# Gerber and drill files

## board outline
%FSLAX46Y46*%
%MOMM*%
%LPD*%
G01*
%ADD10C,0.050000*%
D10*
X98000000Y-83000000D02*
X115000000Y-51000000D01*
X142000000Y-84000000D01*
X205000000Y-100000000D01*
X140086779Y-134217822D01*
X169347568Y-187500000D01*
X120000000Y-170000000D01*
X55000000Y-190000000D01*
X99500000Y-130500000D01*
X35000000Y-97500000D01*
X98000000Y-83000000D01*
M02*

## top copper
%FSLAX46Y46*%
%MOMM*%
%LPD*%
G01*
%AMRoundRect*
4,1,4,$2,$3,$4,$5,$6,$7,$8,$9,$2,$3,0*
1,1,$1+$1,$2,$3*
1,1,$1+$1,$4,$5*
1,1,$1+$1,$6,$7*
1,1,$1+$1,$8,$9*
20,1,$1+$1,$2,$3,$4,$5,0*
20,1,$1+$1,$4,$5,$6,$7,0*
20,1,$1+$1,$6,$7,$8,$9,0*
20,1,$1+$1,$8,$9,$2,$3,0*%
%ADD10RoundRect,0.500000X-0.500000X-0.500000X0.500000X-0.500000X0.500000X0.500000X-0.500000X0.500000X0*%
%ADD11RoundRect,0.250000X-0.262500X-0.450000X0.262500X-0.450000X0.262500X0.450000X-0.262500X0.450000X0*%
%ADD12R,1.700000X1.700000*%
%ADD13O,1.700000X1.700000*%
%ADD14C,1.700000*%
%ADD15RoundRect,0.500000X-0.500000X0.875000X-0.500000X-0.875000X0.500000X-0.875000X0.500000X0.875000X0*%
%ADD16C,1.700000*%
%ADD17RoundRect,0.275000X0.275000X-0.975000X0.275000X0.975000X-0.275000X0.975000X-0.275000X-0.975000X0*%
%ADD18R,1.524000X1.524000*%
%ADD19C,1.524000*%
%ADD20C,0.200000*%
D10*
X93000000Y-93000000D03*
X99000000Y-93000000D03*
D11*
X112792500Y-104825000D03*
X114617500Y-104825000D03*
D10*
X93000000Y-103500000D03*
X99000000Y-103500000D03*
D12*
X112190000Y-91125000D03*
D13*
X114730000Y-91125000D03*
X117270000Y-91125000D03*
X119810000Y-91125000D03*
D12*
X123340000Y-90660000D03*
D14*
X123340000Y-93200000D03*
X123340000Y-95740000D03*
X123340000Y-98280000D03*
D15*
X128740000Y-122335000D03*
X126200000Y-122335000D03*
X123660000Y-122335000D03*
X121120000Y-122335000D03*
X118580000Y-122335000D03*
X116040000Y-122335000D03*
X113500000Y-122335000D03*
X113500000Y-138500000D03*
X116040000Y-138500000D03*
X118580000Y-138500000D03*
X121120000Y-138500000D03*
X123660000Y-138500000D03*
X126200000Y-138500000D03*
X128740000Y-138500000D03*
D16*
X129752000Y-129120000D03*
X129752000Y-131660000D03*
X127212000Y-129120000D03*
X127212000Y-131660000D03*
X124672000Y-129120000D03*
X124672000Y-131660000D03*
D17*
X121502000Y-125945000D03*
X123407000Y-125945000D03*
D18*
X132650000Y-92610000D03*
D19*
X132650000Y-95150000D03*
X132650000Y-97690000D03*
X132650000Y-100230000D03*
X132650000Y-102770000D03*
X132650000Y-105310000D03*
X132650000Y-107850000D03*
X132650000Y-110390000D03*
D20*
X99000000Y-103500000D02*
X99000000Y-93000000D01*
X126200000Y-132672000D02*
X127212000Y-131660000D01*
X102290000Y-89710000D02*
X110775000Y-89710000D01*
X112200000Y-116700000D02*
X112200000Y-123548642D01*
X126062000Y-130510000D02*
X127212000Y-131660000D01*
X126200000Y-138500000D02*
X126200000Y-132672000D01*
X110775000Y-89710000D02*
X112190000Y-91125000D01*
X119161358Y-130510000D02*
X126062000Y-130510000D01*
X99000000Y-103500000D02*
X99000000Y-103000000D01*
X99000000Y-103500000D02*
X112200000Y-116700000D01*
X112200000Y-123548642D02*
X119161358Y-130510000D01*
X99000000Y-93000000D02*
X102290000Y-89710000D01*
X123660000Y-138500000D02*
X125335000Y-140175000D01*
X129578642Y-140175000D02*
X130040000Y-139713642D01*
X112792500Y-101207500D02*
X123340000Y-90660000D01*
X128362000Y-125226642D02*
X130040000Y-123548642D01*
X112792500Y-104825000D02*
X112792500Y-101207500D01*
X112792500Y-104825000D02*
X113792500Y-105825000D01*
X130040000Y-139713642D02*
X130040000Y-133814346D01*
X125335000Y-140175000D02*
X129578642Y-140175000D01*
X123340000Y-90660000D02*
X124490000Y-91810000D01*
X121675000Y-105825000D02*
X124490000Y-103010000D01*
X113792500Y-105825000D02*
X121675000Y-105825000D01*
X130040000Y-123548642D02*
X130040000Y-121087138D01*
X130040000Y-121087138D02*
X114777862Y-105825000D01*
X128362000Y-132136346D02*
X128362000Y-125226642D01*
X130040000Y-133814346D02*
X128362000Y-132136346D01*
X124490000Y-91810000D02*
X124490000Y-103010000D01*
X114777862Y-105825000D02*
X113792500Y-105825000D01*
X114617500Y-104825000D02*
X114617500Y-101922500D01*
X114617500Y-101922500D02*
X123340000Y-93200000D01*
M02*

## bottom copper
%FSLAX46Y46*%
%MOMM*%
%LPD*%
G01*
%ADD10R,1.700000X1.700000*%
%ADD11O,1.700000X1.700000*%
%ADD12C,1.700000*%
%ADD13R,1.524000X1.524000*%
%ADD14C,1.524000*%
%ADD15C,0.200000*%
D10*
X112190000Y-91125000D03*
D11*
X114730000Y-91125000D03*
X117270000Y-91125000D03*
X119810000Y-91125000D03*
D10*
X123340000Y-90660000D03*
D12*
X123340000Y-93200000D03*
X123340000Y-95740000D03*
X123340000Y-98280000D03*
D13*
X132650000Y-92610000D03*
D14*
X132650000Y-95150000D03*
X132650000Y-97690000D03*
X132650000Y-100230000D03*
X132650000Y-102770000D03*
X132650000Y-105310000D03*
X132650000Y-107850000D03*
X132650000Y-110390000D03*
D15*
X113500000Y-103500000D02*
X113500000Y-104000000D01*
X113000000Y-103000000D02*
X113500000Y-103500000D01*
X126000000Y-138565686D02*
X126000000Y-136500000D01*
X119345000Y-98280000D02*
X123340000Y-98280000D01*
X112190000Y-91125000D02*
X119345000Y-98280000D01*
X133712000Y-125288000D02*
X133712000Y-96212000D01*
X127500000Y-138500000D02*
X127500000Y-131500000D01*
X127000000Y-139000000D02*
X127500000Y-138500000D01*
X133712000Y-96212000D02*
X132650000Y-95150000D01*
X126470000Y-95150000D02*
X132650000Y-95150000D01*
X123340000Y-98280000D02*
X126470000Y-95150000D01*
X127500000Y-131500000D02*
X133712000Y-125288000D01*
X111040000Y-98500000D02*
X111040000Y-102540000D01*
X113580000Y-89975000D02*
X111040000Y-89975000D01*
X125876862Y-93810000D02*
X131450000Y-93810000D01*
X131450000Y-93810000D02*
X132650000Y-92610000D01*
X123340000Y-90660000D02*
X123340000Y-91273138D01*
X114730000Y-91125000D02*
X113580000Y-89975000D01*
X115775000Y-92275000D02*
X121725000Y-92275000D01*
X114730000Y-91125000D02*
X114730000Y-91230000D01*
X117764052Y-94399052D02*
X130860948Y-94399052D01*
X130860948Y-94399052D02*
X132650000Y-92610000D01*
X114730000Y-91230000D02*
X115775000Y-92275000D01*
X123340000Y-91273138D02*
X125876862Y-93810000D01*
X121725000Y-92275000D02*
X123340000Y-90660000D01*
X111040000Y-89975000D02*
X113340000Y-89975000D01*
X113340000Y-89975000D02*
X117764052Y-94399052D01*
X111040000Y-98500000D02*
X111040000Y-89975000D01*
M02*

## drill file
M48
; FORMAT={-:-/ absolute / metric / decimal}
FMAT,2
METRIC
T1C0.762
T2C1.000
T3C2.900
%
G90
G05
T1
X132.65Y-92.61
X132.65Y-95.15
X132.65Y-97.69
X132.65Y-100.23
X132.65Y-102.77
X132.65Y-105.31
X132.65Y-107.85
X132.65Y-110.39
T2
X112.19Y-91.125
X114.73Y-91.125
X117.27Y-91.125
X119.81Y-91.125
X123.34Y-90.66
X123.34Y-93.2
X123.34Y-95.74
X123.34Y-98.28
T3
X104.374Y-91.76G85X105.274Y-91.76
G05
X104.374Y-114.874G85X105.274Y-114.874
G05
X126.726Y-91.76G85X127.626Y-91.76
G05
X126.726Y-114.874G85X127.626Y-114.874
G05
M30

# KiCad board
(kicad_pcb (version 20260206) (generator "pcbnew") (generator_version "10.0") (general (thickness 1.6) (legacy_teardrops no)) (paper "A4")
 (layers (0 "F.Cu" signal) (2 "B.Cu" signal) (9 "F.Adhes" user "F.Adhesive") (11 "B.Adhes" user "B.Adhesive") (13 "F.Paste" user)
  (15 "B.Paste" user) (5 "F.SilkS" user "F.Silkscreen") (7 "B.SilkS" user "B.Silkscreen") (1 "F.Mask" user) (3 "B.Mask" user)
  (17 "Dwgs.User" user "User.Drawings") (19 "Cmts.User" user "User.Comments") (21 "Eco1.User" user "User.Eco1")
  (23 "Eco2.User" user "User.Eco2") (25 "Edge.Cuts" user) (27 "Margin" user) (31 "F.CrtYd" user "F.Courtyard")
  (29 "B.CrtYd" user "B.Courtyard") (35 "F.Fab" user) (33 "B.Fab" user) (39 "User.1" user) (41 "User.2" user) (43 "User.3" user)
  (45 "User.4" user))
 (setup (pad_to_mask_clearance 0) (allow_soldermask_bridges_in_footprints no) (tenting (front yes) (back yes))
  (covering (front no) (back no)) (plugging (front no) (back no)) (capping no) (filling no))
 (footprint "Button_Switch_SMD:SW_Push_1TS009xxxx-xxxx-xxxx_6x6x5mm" (layer "F.Cu") (at 96 93)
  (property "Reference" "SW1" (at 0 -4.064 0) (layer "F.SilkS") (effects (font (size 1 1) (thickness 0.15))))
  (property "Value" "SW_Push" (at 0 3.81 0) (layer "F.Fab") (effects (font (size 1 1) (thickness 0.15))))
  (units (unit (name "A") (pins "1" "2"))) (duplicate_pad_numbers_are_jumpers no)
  (pad "1" smd roundrect (at -3 0) (size 2 2) (layers "F.Cu" "F.Mask" "F.Paste") (roundrect_rratio 0.25) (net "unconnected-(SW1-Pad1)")
   (thermal_bridge_angle 45))
  (pad "2" smd roundrect (at 3 0) (size 2 2) (layers "F.Cu" "F.Mask" "F.Paste") (roundrect_rratio 0.25) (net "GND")
   (thermal_bridge_angle 45)))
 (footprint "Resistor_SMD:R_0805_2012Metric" (layer "F.Cu") (at 113.705 104.825)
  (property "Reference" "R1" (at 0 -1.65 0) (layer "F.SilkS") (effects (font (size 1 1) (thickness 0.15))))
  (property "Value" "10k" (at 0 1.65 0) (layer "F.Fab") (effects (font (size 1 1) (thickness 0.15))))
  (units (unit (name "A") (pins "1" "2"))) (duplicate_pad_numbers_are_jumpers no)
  (pad "1" smd roundrect (at -0.9125 0) (size 1.025 1.4) (layers "F.Cu" "F.Mask" "F.Paste") (roundrect_rratio 0.243902) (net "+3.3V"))
  (pad "2" smd roundrect (at 0.9125 0) (size 1.025 1.4) (layers "F.Cu" "F.Mask" "F.Paste") (roundrect_rratio 0.243902) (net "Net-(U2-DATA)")))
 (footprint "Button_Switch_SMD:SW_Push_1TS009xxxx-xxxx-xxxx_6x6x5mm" (layer "F.Cu") (at 96 103.5)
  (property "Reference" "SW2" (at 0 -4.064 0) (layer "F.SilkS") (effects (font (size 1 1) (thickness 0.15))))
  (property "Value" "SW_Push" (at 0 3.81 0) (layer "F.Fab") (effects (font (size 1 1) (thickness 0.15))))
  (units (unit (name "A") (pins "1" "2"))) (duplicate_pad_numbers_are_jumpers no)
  (pad "1" smd roundrect (at -3 0) (size 2 2) (layers "F.Cu" "F.Mask" "F.Paste") (roundrect_rratio 0.25) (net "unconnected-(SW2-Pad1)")
   (thermal_bridge_angle 45))
  (pad "2" smd roundrect (at 3 0) (size 2 2) (layers "F.Cu" "F.Mask" "F.Paste") (roundrect_rratio 0.25) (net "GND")
   (thermal_bridge_angle 45)))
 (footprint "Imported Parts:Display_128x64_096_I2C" (layer "F.Cu") (at 116 91.125)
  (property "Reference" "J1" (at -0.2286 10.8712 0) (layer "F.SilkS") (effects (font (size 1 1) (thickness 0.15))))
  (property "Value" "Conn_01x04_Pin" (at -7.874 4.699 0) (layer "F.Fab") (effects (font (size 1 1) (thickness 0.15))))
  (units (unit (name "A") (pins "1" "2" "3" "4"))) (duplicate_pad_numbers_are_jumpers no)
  (pad "" np_thru_hole oval (at -11.176 0.635) (size 3.8 2.9) (drill oval 3.8 2.9) (layers "*.Cu" "*.Mask"))
  (pad "" np_thru_hole oval (at -11.176 23.749) (size 3.8 2.9) (drill oval 3.8 2.9) (layers "*.Cu" "*.Mask"))
  (pad "" np_thru_hole oval (at 11.176 0.635) (size 3.8 2.9) (drill oval 3.8 2.9) (layers "*.Cu" "*.Mask"))
  (pad "" np_thru_hole oval (at 11.176 23.749) (size 3.8 2.9) (drill oval 3.8 2.9) (layers "*.Cu" "*.Mask"))
  (pad "1" thru_hole rect (at -3.81 0 90) (size 1.7 1.7) (drill 1) (layers "*.Cu" "*.Mask") (remove_unused_layers no) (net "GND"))
  (pad "2" thru_hole oval (at -1.27 0 90) (size 1.7 1.7) (drill 1) (layers "*.Cu" "*.Mask") (remove_unused_layers no) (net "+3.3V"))
  (pad "3" thru_hole oval (at 1.27 0 90) (size 1.7 1.7) (drill 1) (layers "*.Cu" "*.Mask") (remove_unused_layers no)
   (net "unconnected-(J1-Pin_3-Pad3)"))
  (pad "4" thru_hole oval (at 3.81 0 90) (size 1.7 1.7) (drill 1) (layers "*.Cu" "*.Mask") (remove_unused_layers no)
   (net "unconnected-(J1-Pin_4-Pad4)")))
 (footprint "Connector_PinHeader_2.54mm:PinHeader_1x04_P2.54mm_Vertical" (layer "F.Cu") (at 123.34 90.66)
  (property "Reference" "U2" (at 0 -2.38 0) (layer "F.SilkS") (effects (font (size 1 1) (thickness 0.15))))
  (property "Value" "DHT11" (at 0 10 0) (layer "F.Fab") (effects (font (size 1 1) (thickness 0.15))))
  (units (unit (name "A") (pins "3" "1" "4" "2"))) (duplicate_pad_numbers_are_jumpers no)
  (pad "1" thru_hole rect (at 0 0) (size 1.7 1.7) (drill 1) (layers "*.Cu" "*.Mask") (remove_unused_layers no) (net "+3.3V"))
  (pad "2" thru_hole circle (at 0 2.54) (size 1.7 1.7) (drill 1) (layers "*.Cu" "*.Mask") (remove_unused_layers no) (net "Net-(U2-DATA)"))
  (pad "3" thru_hole circle (at 0 5.08) (size 1.7 1.7) (drill 1) (layers "*.Cu" "*.Mask") (remove_unused_layers no)
   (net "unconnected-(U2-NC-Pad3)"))
  (pad "4" thru_hole circle (at 0 7.62) (size 1.7 1.7) (drill 1) (layers "*.Cu" "*.Mask") (remove_unused_layers no) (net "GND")))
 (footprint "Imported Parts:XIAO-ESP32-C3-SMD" (layer "F.Cu") (at 110.62 121.5 -90)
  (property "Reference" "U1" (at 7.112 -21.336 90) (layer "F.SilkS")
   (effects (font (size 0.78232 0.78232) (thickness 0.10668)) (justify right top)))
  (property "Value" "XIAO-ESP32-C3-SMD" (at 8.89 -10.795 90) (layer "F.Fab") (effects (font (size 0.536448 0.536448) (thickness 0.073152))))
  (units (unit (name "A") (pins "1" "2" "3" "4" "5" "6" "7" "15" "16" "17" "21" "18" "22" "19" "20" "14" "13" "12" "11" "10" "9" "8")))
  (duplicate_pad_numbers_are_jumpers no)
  (pad "1" smd roundrect (at 0.835 -18.12 270) (size 2.75 2) (layers "F.Cu" "F.Mask" "F.Paste") (roundrect_rratio 0.25)
   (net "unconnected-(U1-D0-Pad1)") (solder_mask_margin 0.0508) (thermal_bridge_angle 45))
  (pad "2" smd roundrect (at 0.835 -15.58 270) (size 2.75 2) (layers "F.Cu" "F.Mask" "F.Paste") (roundrect_rratio 0.25)
   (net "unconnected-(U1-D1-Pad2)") (solder_mask_margin 0.0508) (thermal_bridge_angle 45))
  (pad "3" smd roundrect (at 0.835 -13.04 270) (size 2.75 2) (layers "F.Cu" "F.Mask" "F.Paste") (roundrect_rratio 0.25)
   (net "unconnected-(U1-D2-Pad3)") (solder_mask_margin 0.0508) (thermal_bridge_angle 45))
  (pad "4" smd roundrect (at 0.835 -10.5 270) (size 2.75 2) (layers "F.Cu" "F.Mask" "F.Paste") (roundrect_rratio 0.25)
   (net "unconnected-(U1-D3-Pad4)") (solder_mask_margin 0.0508) (thermal_bridge_angle 45))
  (pad "5" smd roundrect (at 0.835 -7.96 270) (size 2.75 2) (layers "F.Cu" "F.Mask" "F.Paste") (roundrect_rratio 0.25)
   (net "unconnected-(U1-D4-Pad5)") (solder_mask_margin 0.0508) (thermal_bridge_angle 45))
  (pad "6" smd roundrect (at 0.835 -5.42 270) (size 2.75 2) (layers "F.Cu" "F.Mask" "F.Paste") (roundrect_rratio 0.25)
   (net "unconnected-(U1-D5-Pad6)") (solder_mask_margin 0.0508) (thermal_bridge_angle 45))
  (pad "7" smd roundrect (at 0.835 -2.88 270) (size 2.75 2) (layers "F.Cu" "F.Mask" "F.Paste") (roundrect_rratio 0.25)
   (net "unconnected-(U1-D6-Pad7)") (solder_mask_margin 0.0508) (thermal_bridge_angle 45))
  (pad "8" smd roundrect (at 17 -2.88 270) (size 2.75 2) (layers "F.Cu" "F.Mask" "F.Paste") (roundrect_rratio 0.25)
   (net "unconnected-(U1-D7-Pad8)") (solder_mask_margin 0.0508) (thermal_bridge_angle 45))
  (pad "9" smd roundrect (at 17 -5.42 270) (size 2.75 2) (layers "F.Cu" "F.Mask" "F.Paste") (roundrect_rratio 0.25)
   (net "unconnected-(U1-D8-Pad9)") (solder_mask_margin 0.0508) (thermal_bridge_angle 45))
  (pad "10" smd roundrect (at 17 -7.96 270) (size 2.75 2) (layers "F.Cu" "F.Mask" "F.Paste") (roundrect_rratio 0.25)
   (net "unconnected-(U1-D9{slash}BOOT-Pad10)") (solder_mask_margin 0.0508) (thermal_bridge_angle 45))
  (pad "11" smd roundrect (at 17 -10.5 270) (size 2.75 2) (layers "F.Cu" "F.Mask" "F.Paste") (roundrect_rratio 0.25)
   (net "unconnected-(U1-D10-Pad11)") (solder_mask_margin 0.0508) (thermal_bridge_angle 45))
  (pad "12" smd roundrect (at 17 -13.04 270) (size 2.75 2) (layers "F.Cu" "F.Mask" "F.Paste") (roundrect_rratio 0.25) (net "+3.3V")
   (solder_mask_margin 0.0508) (thermal_bridge_angle 45))
  (pad "13" smd roundrect (at 17 -15.58 270) (size 2.75 2) (layers "F.Cu" "F.Mask" "F.Paste") (roundrect_rratio 0.25) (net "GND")
   (solder_mask_margin 0.0508) (thermal_bridge_angle 45))
  (pad "14" smd roundrect (at 17 -18.12 270) (size 2.75 2) (layers "F.Cu" "F.Mask" "F.Paste") (roundrect_rratio 0.25) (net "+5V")
   (solder_mask_margin 0.0508) (thermal_bridge_angle 45))
  (pad "15" smd circle (at 7.62 -19.132 270) (size 1.7 1.7) (layers "F.Cu" "F.Mask" "F.Paste") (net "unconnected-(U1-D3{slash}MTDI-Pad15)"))
  (pad "16" smd circle (at 10.16 -19.132 270) (size 1.7 1.7) (layers "F.Cu" "F.Mask" "F.Paste") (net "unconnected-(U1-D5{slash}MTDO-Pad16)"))
  (pad "17" smd circle (at 7.62 -16.592 270) (size 1.7 1.7) (layers "F.Cu" "F.Mask" "F.Paste") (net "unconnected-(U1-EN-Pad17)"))
  (pad "18" smd circle (at 10.16 -16.592 270) (size 1.7 1.7) (layers "F.Cu" "F.Mask" "F.Paste") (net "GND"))
  (pad "19" smd circle (at 7.62 -14.052 270) (size 1.7 1.7) (layers "F.Cu" "F.Mask" "F.Paste") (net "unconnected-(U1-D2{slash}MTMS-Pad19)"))
  (pad "20" smd circle (at 10.16 -14.052 270) (size 1.7 1.7) (layers "F.Cu" "F.Mask" "F.Paste") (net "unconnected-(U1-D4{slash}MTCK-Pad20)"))
  (pad "21" smd roundrect (at 4.445 -10.882 90) (size 2.5 1.1) (layers "F.Cu" "F.Mask" "F.Paste") (roundrect_rratio 0.25)
   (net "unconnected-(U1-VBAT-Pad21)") (thermal_bridge_angle 45))
  (pad "22" smd roundrect (at 4.445 -12.787 90) (size 2.5 1.1) (layers "F.Cu" "F.Mask" "F.Paste") (roundrect_rratio 0.25)
   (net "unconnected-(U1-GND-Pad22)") (thermal_bridge_angle 45)))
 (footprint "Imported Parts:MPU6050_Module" (layer "F.Cu") (at 132.65 92.61)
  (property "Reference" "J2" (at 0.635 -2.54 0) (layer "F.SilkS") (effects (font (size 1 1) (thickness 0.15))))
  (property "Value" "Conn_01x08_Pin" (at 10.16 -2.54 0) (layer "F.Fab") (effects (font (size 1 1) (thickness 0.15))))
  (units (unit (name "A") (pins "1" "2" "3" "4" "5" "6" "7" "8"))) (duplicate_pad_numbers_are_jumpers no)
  (pad "1" thru_hole rect (at 0 0) (size 1.524 1.524) (drill 0.762) (layers "*.Cu" "*.Mask") (remove_unused_layers no) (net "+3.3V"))
  (pad "2" thru_hole circle (at 0 2.54) (size 1.524 1.524) (drill 0.762) (layers "*.Cu" "*.Mask") (remove_unused_layers no) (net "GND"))
  (pad "3" thru_hole circle (at 0 5.08) (size 1.524 1.524) (drill 0.762) (layers "*.Cu" "*.Mask") (remove_unused_layers no)
   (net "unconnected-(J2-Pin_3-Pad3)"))
  (pad "4" thru_hole circle (at 0 7.62) (size 1.524 1.524) (drill 0.762) (layers "*.Cu" "*.Mask") (remove_unused_layers no)
   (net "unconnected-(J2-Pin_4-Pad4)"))
  (pad "5" thru_hole circle (at 0 10.16) (size 1.524 1.524) (drill 0.762) (layers "*.Cu" "*.Mask") (remove_unused_layers no)
   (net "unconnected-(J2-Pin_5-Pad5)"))
  (pad "6" thru_hole circle (at 0 12.7) (size 1.524 1.524) (drill 0.762) (layers "*.Cu" "*.Mask") (remove_unused_layers no)
   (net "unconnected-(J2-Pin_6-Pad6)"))
  (pad "7" thru_hole circle (at 0 15.24) (size 1.524 1.524) (drill 0.762) (layers "*.Cu" "*.Mask") (remove_unused_layers no)
   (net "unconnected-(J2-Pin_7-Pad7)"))
  (pad "8" thru_hole circle (at 0 17.78) (size 1.524 1.524) (drill 0.762) (layers "*.Cu" "*.Mask") (remove_unused_layers no)
   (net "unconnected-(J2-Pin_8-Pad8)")))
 (gr_poly
  (pts (xy 98 83) (xy 115 51) (xy 142 84) (xy 205 100) (xy 140.086779 134.217822) (xy 169.347568 187.5) (xy 120 170) (xy 55 190)
   (xy 99.5 130.5) (xy 35 97.5))
  (stroke (width 0.05) (type solid)) (fill no) (locked yes) (layer "Edge.Cuts"))
 (segment (start 113.5 103.5) (end 113.5 104) (width 0.2) (layer "B.Cu") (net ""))
 (segment (start 113 103) (end 113.5 103.5) (width 0.2) (layer "B.Cu") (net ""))
 (segment (start 126 138.565686) (end 126 136.5) (width 0.2) (layer "B.Cu") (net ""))
 (segment (start 99 103.5) (end 99 93) (width 0.2) (layer "F.Cu") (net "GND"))
 (segment (start 126.2 132.672) (end 127.212 131.66) (width 0.2) (layer "F.Cu") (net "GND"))
 (segment (start 102.29 89.71) (end 110.775 89.71) (width 0.2) (layer "F.Cu") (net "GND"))
 (segment (start 112.2 116.7) (end 112.2 123.548642) (width 0.2) (layer "F.Cu") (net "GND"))
 (segment (start 126.062 130.51) (end 127.212 131.66) (width 0.2) (layer "F.Cu") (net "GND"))
 (segment (start 126.2 138.5) (end 126.2 132.672) (width 0.2) (layer "F.Cu") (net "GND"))
 (segment (start 110.775 89.71) (end 112.19 91.125) (width 0.2) (layer "F.Cu") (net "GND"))
 (segment (start 119.161358 130.51) (end 126.062 130.51) (width 0.2) (layer "F.Cu") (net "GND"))
 (segment (start 99 103.5) (end 99 103) (width 0.2) (layer "F.Cu") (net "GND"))
 (segment (start 99 103.5) (end 112.2 116.7) (width 0.2) (layer "F.Cu") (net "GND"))
 (segment (start 112.2 123.548642) (end 119.161358 130.51) (width 0.2) (layer "F.Cu") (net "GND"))
 (segment (start 99 93) (end 102.29 89.71) (width 0.2) (layer "F.Cu") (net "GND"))
 (segment (start 119.345 98.28) (end 123.34 98.28) (width 0.2) (layer "B.Cu") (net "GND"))
 (segment (start 112.19 91.125) (end 119.345 98.28) (width 0.2) (layer "B.Cu") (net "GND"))
 (segment (start 133.712 125.288) (end 133.712 96.212) (width 0.2) (layer "B.Cu") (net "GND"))
 (segment (start 127.5 138.5) (end 127.5 131.5) (width 0.2) (layer "B.Cu") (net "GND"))
 (segment (start 127 139) (end 127.5 138.5) (width 0.2) (layer "B.Cu") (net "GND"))
 (segment (start 133.712 96.212) (end 132.65 95.15) (width 0.2) (layer "B.Cu") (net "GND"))
 (segment (start 126.47 95.15) (end 132.65 95.15) (width 0.2) (layer "B.Cu") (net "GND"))
 (segment (start 123.34 98.28) (end 126.47 95.15) (width 0.2) (layer "B.Cu") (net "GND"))
 (segment (start 127.5 131.5) (end 133.712 125.288) (width 0.2) (layer "B.Cu") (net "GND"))
 (segment (start 123.66 138.5) (end 125.335 140.175) (width 0.2) (layer "F.Cu") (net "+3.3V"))
 (segment (start 129.578642 140.175) (end 130.04 139.713642) (width 0.2) (layer "F.Cu") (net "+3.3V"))
 (segment (start 112.7925 101.2075) (end 123.34 90.66) (width 0.2) (layer "F.Cu") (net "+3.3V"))
 (segment (start 128.362 125.226642) (end 130.04 123.548642) (width 0.2) (layer "F.Cu") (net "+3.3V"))
 (segment (start 112.7925 104.825) (end 112.7925 101.2075) (width 0.2) (layer "F.Cu") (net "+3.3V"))
 (segment (start 112.7925 104.825) (end 113.7925 105.825) (width 0.2) (layer "F.Cu") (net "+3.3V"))
 (segment (start 130.04 139.713642) (end 130.04 133.814346) (width 0.2) (layer "F.Cu") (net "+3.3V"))
 (segment (start 125.335 140.175) (end 129.578642 140.175) (width 0.2) (layer "F.Cu") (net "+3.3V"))
 (segment (start 123.34 90.66) (end 124.49 91.81) (width 0.2) (layer "F.Cu") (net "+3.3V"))
 (segment (start 121.675 105.825) (end 124.49 103.01) (width 0.2) (layer "F.Cu") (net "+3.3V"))
 (segment (start 113.7925 105.825) (end 121.675 105.825) (width 0.2) (layer "F.Cu") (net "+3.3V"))
 (segment (start 130.04 123.548642) (end 130.04 121.087138) (width 0.2) (layer "F.Cu") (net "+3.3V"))
 (segment (start 130.04 121.087138) (end 114.777862 105.825) (width 0.2) (layer "F.Cu") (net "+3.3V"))
 (segment (start 128.362 132.136346) (end 128.362 125.226642) (width 0.2) (layer "F.Cu") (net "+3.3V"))
 (segment (start 130.04 133.814346) (end 128.362 132.136346) (width 0.2) (layer "F.Cu") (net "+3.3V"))
 (segment (start 124.49 91.81) (end 124.49 103.01) (width 0.2) (layer "F.Cu") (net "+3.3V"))
 (segment (start 114.777862 105.825) (end 113.7925 105.825) (width 0.2) (layer "F.Cu") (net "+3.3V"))
 (segment (start 111.04 98.5) (end 111.04 102.54) (width 0.2) (layer "B.Cu") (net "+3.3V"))
 (segment (start 113.58 89.975) (end 111.04 89.975) (width 0.2) (layer "B.Cu") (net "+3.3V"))
 (segment (start 125.876862 93.81) (end 131.45 93.81) (width 0.2) (layer "B.Cu") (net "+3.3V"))
 (segment (start 131.45 93.81) (end 132.65 92.61) (width 0.2) (layer "B.Cu") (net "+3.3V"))
 (segment (start 123.34 90.66) (end 123.34 91.273138) (width 0.2) (layer "B.Cu") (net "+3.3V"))
 (segment (start 114.73 91.125) (end 113.58 89.975) (width 0.2) (layer "B.Cu") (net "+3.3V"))
 (segment (start 115.775 92.275) (end 121.725 92.275) (width 0.2) (layer "B.Cu") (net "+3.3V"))
 (segment (start 114.73 91.125) (end 114.73 91.23) (width 0.2) (layer "B.Cu") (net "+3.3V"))
 (segment (start 117.764052 94.399052) (end 130.860948 94.399052) (width 0.2) (layer "B.Cu") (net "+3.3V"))
 (segment (start 130.860948 94.399052) (end 132.65 92.61) (width 0.2) (layer "B.Cu") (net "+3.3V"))
 (segment (start 114.73 91.23) (end 115.775 92.275) (width 0.2) (layer "B.Cu") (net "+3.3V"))
 (segment (start 123.34 91.273138) (end 125.876862 93.81) (width 0.2) (layer "B.Cu") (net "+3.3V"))
 (segment (start 121.725 92.275) (end 123.34 90.66) (width 0.2) (layer "B.Cu") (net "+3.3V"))
 (segment (start 111.04 89.975) (end 113.34 89.975) (width 0.2) (layer "B.Cu") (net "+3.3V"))
 (segment (start 113.34 89.975) (end 117.764052 94.399052) (width 0.2) (layer "B.Cu") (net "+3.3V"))
 (segment (start 111.04 98.5) (end 111.04 89.975) (width 0.2) (layer "B.Cu") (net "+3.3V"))
 (segment (start 114.6175 104.825) (end 114.6175 101.9225) (width 0.2) (layer "F.Cu") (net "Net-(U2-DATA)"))
 (segment (start 114.6175 101.9225) (end 123.34 93.2) (width 0.2) (layer "F.Cu") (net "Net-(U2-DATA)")))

